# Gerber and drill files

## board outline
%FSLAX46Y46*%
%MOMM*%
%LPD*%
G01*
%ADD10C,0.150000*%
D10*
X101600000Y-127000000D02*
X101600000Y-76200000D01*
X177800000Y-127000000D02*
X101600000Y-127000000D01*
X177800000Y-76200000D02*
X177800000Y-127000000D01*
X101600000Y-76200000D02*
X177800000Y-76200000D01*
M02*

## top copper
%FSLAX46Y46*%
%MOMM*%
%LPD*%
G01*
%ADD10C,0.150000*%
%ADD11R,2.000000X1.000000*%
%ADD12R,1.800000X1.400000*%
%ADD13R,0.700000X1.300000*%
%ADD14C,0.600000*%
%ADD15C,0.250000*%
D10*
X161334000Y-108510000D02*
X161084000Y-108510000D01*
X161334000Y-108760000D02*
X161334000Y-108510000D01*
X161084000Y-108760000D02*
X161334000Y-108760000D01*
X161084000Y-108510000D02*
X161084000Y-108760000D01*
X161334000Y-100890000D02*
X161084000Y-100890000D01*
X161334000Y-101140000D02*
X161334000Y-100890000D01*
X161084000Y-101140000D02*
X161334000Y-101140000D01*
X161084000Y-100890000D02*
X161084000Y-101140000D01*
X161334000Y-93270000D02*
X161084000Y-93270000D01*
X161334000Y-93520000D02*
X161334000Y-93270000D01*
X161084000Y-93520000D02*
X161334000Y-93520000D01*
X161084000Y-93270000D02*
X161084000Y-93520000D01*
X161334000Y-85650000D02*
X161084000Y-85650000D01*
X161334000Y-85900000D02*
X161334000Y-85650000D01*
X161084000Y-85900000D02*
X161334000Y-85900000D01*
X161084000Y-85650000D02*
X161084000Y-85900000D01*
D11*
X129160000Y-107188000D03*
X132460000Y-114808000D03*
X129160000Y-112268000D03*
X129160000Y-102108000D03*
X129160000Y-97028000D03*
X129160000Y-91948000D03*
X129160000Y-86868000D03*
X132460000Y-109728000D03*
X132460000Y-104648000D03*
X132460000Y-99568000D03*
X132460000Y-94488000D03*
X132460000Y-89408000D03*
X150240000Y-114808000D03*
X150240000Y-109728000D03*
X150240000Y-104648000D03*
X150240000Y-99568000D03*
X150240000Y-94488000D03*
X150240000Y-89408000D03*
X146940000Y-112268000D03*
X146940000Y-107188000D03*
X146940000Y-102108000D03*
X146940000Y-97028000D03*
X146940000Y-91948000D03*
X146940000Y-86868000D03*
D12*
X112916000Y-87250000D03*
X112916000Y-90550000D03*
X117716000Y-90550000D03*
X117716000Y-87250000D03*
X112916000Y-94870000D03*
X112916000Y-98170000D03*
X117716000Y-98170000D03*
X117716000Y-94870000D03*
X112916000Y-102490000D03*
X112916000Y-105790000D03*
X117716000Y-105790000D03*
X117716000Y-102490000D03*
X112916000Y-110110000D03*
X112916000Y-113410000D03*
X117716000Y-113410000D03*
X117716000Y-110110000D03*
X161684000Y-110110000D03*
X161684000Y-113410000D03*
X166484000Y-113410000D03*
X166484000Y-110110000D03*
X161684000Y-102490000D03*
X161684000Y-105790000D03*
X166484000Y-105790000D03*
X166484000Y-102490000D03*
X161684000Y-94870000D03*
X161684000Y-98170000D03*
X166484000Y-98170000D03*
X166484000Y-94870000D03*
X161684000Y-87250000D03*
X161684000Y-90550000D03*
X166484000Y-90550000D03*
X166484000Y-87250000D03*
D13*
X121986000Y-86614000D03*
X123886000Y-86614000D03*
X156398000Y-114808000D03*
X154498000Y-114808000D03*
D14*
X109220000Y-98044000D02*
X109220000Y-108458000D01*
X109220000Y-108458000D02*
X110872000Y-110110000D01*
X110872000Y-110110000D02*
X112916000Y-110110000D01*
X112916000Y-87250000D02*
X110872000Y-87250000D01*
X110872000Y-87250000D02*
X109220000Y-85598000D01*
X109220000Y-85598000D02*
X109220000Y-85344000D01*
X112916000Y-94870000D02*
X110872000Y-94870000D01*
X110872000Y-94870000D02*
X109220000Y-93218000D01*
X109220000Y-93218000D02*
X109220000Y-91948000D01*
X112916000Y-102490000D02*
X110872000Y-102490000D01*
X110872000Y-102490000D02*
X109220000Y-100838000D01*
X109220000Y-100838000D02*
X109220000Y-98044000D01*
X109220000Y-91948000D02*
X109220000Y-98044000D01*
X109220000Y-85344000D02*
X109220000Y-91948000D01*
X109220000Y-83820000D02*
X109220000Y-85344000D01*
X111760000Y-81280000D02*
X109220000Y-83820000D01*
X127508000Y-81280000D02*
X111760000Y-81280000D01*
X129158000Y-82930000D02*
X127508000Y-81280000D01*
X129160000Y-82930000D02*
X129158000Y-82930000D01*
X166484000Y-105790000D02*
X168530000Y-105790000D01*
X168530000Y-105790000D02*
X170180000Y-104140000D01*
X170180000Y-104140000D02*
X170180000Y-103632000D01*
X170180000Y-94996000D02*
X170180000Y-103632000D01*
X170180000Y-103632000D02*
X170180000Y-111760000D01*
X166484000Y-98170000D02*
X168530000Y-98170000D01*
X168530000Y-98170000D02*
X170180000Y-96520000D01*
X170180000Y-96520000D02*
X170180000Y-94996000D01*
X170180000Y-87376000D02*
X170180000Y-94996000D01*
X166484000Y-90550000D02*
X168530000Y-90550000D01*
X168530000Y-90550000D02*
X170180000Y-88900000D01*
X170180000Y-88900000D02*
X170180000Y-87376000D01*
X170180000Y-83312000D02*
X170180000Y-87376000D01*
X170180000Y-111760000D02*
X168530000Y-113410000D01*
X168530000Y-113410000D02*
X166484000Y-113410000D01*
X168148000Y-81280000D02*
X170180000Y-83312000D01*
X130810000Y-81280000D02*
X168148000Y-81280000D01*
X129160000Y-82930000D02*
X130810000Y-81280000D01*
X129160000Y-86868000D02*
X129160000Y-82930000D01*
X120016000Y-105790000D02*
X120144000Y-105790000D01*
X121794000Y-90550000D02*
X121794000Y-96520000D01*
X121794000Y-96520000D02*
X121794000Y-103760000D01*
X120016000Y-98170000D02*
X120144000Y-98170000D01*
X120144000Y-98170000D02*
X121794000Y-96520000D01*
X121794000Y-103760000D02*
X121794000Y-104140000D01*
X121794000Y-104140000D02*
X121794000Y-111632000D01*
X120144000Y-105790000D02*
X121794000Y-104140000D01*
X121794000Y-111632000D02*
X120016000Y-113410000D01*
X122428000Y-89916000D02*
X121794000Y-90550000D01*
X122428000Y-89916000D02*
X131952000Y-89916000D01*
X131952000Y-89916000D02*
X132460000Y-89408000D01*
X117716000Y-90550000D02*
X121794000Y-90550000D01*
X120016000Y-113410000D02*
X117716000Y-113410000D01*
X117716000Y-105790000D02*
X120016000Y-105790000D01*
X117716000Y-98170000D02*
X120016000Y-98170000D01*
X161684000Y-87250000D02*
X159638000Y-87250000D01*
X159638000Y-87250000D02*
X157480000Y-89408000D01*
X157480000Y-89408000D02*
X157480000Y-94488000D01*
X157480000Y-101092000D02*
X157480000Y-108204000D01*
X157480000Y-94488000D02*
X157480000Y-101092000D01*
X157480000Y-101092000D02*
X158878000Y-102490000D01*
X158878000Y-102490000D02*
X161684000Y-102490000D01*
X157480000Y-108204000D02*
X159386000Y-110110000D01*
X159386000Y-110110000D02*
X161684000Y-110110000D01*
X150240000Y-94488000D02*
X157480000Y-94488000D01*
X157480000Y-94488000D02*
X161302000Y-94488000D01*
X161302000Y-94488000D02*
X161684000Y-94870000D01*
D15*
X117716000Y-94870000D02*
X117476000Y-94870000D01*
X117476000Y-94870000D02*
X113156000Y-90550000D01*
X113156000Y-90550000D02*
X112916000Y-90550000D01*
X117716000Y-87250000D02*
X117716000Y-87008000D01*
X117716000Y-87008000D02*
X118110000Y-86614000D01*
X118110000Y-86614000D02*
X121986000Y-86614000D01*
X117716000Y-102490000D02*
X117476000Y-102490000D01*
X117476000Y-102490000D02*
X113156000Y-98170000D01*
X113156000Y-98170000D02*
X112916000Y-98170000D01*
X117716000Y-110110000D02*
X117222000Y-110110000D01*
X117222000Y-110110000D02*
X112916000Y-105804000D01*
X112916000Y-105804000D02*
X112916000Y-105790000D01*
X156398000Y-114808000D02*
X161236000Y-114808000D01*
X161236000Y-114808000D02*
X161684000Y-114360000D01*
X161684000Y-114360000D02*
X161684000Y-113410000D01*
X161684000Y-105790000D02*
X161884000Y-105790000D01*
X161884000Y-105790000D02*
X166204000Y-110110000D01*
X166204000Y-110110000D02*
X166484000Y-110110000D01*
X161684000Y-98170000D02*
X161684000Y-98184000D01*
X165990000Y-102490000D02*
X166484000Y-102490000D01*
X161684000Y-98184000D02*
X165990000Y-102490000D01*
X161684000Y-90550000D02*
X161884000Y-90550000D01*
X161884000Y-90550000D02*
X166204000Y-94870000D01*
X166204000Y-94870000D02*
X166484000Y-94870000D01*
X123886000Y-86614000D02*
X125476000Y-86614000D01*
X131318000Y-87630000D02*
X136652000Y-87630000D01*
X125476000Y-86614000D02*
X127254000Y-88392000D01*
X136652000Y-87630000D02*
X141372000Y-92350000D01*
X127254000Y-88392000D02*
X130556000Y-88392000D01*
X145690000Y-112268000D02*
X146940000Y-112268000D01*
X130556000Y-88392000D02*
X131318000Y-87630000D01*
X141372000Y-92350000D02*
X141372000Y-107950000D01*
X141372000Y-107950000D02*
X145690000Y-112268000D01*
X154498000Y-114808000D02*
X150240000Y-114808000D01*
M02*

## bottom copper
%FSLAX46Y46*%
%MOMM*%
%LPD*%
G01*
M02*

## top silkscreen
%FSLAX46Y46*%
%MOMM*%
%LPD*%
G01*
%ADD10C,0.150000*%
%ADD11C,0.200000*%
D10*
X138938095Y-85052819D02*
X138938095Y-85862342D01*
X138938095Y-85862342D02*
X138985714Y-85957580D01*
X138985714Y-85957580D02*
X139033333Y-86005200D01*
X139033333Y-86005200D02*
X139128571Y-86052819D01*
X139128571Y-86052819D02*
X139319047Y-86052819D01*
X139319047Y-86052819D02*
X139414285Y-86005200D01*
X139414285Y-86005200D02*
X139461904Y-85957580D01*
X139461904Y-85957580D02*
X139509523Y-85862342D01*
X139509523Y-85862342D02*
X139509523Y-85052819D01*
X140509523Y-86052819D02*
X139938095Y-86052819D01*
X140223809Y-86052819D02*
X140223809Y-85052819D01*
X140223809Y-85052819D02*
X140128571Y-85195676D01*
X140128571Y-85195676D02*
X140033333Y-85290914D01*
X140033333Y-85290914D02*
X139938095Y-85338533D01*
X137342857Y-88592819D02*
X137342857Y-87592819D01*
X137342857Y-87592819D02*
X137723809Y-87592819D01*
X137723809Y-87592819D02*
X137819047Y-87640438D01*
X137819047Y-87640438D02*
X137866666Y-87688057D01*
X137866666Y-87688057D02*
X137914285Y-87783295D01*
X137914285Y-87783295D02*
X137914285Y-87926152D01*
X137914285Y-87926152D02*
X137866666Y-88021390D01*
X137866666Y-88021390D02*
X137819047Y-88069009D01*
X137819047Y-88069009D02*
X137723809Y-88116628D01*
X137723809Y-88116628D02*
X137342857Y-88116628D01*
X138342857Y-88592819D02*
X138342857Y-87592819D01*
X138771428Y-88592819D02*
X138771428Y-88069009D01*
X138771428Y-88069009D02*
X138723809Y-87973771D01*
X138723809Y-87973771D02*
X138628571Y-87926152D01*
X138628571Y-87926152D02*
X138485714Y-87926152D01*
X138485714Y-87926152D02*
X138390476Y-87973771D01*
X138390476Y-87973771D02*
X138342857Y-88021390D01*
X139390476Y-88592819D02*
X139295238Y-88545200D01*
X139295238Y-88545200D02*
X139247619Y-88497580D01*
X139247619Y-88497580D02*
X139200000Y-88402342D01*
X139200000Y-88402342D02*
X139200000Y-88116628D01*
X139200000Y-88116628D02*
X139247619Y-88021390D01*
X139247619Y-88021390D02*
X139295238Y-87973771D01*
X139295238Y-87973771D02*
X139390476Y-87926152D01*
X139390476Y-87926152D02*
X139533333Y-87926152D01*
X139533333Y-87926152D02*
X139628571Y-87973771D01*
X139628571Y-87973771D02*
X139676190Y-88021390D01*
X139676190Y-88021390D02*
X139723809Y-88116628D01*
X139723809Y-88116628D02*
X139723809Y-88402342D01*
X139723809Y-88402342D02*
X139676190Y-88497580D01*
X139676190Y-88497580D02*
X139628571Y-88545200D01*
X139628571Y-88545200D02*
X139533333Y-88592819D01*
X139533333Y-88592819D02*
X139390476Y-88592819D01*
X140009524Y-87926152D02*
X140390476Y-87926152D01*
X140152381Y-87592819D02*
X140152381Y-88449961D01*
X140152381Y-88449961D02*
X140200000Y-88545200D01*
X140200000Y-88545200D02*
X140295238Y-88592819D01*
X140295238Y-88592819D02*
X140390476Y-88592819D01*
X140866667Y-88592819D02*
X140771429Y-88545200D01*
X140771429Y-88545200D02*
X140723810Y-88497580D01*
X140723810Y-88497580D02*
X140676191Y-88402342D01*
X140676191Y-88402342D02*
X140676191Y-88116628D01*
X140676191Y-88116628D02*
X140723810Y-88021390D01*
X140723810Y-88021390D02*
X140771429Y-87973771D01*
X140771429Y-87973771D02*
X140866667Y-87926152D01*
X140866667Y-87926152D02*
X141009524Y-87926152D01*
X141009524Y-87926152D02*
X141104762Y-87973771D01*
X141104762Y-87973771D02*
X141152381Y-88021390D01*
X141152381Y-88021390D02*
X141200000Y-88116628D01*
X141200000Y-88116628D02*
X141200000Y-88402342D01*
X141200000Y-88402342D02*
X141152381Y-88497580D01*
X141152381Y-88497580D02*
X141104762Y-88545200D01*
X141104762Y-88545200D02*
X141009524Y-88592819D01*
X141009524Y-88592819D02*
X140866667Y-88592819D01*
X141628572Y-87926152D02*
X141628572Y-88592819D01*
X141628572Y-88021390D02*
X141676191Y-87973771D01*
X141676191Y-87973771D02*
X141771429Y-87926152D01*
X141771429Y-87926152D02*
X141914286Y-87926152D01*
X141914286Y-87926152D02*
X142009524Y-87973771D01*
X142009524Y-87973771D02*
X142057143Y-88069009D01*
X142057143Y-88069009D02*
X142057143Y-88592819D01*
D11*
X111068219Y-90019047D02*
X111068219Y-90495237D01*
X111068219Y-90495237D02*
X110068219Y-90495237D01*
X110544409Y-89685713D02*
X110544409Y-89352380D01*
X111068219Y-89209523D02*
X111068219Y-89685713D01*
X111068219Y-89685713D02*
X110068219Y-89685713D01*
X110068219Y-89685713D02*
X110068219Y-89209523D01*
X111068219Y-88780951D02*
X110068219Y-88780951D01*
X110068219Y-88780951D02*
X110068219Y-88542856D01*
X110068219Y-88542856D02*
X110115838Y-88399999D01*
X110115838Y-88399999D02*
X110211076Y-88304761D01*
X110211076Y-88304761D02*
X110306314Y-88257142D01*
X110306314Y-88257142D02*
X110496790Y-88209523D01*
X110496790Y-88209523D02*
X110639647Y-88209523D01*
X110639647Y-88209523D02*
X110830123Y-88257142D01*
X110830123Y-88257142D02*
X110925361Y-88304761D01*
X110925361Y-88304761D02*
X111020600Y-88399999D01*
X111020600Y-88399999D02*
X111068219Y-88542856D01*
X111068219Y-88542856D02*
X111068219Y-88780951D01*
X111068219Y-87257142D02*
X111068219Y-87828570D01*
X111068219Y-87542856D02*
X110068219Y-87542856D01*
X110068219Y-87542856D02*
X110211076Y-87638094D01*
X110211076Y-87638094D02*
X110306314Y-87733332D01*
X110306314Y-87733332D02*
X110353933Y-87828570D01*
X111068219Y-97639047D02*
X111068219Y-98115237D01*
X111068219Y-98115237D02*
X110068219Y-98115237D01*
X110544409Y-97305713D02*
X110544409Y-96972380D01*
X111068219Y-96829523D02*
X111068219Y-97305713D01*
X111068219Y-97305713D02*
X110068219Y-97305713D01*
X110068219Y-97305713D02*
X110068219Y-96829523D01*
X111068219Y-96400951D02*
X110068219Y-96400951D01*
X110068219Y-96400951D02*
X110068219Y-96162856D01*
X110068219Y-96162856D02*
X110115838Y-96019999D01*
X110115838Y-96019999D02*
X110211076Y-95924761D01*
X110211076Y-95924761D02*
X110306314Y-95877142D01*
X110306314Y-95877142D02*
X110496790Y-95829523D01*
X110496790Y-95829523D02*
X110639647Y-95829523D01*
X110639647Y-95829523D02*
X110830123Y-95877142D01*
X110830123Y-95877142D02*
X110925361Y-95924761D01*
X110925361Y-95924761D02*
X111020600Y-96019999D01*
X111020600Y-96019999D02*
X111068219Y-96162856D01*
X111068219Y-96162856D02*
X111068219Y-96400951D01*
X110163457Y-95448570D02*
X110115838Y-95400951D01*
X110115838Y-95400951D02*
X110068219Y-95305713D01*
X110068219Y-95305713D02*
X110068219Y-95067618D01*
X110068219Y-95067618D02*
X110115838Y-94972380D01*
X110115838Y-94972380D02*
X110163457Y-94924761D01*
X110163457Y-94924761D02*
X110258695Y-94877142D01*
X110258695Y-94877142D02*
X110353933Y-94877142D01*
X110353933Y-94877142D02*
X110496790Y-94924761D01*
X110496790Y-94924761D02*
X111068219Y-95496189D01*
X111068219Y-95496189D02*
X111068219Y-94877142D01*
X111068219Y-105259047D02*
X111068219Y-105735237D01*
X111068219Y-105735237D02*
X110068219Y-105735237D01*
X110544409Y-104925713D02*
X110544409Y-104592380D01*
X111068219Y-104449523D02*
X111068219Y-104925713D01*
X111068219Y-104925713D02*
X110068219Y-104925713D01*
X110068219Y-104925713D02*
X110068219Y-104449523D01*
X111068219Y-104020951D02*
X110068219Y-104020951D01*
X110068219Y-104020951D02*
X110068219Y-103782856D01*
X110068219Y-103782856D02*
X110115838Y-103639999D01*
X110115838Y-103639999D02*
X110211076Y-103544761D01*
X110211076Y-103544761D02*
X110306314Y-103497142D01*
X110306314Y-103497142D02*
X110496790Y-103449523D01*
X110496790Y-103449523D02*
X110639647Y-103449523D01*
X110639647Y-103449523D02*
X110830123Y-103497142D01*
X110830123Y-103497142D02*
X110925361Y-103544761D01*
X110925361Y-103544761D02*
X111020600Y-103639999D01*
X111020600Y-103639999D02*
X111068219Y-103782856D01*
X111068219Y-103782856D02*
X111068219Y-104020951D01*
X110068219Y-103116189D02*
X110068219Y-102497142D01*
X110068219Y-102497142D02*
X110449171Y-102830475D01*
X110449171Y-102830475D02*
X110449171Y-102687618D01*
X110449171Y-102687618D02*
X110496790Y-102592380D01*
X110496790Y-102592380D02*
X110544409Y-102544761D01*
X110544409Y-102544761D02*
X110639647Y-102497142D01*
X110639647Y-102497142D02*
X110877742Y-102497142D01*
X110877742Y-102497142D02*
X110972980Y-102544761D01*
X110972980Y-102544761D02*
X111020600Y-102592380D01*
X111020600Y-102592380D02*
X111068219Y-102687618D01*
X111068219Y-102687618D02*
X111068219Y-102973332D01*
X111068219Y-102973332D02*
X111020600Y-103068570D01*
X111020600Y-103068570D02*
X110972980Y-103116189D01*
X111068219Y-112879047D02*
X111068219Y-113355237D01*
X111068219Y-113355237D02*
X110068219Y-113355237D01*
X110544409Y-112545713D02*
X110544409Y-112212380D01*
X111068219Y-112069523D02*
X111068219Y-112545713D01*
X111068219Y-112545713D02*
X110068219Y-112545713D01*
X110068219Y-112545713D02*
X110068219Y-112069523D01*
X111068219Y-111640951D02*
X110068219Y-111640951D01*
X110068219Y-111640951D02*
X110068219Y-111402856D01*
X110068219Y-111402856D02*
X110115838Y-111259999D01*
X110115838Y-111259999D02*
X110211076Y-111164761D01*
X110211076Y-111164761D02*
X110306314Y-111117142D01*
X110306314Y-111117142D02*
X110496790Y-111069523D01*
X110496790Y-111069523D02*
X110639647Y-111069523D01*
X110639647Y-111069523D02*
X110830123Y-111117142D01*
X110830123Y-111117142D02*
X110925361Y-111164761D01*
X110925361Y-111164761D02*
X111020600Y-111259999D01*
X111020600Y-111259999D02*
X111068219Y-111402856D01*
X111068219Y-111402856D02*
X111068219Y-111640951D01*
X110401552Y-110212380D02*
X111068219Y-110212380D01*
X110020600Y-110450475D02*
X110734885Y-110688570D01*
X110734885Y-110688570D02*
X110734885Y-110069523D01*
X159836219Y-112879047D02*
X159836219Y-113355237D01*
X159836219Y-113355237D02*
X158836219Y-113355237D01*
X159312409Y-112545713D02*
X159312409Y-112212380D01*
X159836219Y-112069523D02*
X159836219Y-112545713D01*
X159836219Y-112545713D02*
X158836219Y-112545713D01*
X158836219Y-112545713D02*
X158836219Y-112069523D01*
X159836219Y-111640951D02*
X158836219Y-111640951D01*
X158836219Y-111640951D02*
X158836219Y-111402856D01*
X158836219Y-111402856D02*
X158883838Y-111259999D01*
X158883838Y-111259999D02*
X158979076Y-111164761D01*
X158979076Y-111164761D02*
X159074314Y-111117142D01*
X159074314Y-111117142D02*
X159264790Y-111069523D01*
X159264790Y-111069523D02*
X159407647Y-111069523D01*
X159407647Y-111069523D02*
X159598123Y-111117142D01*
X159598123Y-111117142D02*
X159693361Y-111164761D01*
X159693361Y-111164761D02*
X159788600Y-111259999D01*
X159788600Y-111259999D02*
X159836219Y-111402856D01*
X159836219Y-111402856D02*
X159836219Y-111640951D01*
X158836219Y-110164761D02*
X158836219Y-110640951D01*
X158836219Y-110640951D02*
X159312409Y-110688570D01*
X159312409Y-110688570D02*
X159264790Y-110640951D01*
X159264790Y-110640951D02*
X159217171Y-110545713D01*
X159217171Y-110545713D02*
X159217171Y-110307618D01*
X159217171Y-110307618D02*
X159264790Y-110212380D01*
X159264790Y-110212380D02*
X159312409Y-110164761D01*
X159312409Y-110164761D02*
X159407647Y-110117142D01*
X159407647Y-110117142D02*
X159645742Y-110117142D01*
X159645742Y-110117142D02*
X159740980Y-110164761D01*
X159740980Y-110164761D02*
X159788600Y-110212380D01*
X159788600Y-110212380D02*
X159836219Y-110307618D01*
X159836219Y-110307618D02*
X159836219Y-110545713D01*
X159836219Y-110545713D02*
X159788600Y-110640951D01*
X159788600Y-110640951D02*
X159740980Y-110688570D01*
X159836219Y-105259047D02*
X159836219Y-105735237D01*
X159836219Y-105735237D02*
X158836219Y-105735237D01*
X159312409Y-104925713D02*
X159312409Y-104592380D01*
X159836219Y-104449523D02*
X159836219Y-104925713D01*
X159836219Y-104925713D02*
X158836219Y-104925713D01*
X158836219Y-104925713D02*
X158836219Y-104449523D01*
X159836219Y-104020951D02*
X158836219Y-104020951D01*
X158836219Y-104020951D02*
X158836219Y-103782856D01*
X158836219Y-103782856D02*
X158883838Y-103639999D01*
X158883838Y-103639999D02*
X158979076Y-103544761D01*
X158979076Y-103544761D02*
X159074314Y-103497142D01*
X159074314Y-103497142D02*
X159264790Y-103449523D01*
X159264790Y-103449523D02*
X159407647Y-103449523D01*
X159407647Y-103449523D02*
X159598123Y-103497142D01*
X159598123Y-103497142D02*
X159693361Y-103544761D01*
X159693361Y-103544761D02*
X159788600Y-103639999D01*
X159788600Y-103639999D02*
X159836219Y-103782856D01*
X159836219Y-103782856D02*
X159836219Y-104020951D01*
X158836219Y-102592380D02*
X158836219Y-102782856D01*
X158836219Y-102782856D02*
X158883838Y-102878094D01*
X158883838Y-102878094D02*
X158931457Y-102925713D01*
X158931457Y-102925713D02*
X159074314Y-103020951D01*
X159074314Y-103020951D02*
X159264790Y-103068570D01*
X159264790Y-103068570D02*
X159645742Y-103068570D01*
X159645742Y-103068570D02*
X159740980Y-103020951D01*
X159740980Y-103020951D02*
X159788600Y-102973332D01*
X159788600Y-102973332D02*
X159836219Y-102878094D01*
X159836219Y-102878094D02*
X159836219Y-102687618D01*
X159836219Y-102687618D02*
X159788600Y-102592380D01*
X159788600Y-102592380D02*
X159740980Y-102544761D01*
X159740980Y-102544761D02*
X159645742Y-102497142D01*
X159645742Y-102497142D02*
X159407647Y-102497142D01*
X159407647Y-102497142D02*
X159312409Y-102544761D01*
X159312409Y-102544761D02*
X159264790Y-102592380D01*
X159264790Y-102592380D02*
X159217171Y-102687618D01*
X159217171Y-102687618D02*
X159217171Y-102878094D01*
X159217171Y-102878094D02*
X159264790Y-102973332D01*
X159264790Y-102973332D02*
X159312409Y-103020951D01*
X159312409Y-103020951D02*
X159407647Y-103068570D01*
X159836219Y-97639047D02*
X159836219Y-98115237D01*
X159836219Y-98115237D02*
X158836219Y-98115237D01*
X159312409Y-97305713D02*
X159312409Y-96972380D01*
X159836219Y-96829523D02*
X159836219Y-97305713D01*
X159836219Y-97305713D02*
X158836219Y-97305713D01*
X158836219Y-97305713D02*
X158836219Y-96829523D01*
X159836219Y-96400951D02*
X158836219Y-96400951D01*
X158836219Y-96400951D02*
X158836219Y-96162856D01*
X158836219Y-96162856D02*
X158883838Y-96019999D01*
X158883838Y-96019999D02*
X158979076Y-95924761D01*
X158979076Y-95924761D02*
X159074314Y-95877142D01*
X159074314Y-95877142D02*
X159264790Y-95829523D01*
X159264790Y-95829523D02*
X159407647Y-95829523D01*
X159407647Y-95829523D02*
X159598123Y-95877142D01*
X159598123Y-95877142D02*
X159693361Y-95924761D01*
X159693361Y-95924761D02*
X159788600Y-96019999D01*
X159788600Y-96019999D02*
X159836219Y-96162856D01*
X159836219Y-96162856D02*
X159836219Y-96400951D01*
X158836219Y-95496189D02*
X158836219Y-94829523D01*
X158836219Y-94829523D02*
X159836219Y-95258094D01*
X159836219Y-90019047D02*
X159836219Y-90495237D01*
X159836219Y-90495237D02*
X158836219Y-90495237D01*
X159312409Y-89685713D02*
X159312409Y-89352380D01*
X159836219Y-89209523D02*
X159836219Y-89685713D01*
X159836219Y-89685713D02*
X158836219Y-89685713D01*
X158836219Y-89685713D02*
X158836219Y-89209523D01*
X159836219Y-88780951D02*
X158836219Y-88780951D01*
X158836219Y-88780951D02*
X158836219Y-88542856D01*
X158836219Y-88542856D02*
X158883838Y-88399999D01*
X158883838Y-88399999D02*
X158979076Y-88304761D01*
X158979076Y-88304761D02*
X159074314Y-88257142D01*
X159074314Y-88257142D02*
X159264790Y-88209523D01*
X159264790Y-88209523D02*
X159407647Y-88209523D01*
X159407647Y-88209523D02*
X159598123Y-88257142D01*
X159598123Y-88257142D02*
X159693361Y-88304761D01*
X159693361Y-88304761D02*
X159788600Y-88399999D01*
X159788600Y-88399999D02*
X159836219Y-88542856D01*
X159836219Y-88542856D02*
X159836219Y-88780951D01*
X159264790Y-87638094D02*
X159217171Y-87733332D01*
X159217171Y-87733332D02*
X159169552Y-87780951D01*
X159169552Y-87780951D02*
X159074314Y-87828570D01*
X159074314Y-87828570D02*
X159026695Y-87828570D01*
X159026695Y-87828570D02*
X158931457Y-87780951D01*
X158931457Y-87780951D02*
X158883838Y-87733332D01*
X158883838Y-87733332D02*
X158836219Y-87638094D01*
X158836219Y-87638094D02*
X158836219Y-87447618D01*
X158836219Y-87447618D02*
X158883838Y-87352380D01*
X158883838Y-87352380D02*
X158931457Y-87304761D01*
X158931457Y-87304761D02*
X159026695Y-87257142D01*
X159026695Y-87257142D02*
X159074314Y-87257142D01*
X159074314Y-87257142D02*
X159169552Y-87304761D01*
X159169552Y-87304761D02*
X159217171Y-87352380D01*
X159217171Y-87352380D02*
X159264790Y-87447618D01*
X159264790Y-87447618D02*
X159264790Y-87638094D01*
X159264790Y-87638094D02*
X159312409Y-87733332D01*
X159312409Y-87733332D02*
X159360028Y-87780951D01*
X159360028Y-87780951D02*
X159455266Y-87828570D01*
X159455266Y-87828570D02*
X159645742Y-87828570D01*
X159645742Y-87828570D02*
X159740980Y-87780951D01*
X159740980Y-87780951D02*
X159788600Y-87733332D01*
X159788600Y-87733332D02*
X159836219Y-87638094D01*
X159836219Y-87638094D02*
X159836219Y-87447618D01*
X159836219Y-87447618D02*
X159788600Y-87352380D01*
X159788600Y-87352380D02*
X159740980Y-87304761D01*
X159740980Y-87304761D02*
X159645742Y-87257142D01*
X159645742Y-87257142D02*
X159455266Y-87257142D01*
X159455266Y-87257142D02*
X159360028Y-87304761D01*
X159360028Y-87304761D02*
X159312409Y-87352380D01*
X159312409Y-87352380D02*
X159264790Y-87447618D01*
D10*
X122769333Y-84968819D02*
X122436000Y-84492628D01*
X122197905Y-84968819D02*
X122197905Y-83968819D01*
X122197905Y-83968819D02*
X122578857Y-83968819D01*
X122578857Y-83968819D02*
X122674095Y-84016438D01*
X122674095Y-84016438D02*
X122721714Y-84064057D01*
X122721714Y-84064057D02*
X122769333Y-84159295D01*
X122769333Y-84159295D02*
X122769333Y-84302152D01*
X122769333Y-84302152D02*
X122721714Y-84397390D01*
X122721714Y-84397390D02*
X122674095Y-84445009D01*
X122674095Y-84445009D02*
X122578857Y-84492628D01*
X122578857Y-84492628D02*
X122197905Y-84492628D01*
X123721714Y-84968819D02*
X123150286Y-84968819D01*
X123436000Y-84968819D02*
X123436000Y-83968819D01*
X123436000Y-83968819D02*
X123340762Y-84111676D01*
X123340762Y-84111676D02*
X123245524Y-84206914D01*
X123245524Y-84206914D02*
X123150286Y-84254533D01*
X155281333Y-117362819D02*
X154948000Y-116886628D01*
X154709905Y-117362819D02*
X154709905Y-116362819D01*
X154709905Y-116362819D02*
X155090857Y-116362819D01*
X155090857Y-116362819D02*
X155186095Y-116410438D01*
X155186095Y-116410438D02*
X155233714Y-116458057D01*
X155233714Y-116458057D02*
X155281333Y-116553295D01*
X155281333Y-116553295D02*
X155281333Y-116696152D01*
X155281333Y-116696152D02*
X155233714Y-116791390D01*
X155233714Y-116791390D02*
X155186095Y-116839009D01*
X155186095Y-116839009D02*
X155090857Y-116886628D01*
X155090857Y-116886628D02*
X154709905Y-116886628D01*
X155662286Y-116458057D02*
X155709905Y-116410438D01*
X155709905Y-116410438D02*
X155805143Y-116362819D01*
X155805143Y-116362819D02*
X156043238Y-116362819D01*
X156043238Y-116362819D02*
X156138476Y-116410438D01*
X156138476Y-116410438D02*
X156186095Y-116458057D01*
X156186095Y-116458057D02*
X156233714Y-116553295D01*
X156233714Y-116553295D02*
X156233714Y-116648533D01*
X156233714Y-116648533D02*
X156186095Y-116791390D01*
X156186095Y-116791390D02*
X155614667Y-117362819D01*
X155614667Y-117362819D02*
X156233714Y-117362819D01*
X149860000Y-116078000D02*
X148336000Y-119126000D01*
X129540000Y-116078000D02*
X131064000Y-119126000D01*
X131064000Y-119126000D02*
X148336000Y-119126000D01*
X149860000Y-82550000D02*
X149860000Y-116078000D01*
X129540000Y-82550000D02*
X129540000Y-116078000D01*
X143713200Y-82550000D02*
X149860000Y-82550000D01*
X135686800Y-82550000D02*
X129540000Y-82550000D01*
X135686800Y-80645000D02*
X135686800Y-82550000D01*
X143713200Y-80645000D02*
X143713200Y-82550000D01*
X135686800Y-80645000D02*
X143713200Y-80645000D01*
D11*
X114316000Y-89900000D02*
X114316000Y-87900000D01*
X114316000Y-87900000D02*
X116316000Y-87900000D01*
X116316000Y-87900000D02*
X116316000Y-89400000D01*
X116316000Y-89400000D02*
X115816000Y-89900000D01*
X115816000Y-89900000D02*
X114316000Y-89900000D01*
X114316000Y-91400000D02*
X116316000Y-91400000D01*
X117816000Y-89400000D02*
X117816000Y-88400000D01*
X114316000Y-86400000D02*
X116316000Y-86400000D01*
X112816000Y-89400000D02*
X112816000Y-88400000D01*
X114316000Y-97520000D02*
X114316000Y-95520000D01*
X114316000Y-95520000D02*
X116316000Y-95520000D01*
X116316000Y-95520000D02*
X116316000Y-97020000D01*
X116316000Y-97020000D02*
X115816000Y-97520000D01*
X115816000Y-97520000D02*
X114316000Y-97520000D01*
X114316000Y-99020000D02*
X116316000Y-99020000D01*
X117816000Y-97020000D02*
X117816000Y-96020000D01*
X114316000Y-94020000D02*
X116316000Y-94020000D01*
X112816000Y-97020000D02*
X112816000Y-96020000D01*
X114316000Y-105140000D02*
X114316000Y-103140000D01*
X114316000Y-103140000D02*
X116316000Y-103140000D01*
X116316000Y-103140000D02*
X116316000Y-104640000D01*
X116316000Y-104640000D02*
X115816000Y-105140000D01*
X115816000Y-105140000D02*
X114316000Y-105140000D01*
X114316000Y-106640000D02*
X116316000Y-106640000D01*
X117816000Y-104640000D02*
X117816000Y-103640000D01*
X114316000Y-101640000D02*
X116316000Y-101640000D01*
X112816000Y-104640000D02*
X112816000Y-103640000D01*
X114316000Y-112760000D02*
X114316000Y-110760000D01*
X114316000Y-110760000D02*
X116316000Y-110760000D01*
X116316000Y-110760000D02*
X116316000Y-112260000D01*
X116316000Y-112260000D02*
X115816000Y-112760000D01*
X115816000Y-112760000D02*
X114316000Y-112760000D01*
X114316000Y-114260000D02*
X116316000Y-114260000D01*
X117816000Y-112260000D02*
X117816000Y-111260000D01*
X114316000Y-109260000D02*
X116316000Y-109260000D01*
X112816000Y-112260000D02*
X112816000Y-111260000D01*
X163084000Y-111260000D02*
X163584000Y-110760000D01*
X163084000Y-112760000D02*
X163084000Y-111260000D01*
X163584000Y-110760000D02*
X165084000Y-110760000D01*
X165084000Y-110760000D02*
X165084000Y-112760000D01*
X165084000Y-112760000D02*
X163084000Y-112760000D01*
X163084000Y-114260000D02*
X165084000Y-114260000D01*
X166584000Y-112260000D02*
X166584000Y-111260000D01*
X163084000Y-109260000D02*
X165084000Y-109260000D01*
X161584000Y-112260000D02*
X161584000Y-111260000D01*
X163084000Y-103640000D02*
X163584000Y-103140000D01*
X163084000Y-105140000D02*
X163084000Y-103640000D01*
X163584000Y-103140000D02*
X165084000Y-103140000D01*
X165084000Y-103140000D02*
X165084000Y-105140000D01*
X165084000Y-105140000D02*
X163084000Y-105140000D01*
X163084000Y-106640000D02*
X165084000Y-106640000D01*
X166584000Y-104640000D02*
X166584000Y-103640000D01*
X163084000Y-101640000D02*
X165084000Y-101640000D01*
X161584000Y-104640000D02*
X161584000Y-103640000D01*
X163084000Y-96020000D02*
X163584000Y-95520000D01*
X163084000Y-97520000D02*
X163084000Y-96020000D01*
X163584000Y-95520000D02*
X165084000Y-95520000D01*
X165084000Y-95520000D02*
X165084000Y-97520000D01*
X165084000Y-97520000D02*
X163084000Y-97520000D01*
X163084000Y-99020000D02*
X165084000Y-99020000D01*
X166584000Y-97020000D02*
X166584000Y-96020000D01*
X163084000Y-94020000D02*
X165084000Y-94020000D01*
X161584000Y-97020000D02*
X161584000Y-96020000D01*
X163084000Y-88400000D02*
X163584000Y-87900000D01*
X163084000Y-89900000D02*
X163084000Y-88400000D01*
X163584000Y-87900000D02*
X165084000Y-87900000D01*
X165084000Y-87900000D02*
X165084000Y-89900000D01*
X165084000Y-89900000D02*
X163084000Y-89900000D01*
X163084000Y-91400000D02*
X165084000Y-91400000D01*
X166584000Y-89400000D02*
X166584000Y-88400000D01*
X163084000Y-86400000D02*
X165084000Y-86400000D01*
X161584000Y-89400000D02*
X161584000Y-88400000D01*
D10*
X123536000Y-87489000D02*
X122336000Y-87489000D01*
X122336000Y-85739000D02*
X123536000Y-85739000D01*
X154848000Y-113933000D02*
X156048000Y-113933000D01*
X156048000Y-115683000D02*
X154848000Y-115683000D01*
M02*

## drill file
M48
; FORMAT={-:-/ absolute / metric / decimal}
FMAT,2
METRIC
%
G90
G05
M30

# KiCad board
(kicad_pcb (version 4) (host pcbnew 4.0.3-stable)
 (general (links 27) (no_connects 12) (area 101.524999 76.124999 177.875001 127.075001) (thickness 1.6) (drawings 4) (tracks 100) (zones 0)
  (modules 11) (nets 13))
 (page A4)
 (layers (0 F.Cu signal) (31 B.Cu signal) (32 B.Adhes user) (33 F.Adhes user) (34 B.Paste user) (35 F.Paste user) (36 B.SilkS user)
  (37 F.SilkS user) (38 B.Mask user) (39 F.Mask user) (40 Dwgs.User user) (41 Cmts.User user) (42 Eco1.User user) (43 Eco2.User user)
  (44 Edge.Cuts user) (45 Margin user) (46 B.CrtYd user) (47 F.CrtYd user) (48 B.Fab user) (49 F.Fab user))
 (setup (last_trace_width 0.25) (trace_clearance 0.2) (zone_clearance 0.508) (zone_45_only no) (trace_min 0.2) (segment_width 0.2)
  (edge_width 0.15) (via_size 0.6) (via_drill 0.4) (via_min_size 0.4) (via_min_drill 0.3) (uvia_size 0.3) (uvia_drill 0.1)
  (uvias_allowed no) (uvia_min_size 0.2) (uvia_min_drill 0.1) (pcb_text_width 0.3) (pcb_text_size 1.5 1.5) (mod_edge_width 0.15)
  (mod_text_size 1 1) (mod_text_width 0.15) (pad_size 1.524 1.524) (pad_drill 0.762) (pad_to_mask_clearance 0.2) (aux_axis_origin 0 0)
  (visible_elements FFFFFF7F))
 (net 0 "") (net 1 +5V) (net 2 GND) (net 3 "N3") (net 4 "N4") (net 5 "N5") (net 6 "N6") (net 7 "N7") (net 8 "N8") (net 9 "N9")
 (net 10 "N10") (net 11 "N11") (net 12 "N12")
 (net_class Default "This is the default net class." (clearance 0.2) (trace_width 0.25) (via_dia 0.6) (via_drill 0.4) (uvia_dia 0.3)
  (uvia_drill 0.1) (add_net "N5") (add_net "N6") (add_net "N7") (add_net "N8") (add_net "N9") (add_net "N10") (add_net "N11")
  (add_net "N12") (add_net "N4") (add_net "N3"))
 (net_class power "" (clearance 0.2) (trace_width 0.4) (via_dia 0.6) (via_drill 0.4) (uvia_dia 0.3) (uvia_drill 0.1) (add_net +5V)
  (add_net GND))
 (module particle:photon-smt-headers (layer F.Cu) (at 139.7 102.108)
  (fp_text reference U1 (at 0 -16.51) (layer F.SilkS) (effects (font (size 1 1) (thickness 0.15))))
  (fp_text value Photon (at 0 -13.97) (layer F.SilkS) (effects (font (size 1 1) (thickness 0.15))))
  (fp_line (start 10.16 13.97) (end 8.636 17.018) (layer F.SilkS) (width 0.15))
  (fp_line (start -10.16 13.97) (end -8.636 17.018) (layer F.SilkS) (width 0.15))
  (fp_line (start -8.636 17.018) (end 8.636 17.018) (layer F.SilkS) (width 0.15))
  (fp_line (start 10.16 -19.558) (end 10.16 13.97) (layer F.SilkS) (width 0.15))
  (fp_line (start -10.16 -19.558) (end -10.16 13.97) (layer F.SilkS) (width 0.15))
  (fp_line (start 4.0132 -19.558) (end 10.16 -19.558) (layer F.SilkS) (width 0.15))
  (fp_line (start -4.0132 -19.558) (end -10.16 -19.558) (layer F.SilkS) (width 0.15))
  (fp_line (start -4.0132 -21.463) (end -4.0132 -19.558) (layer F.SilkS) (width 0.15))
  (fp_line (start 4.0132 -21.463) (end 4.0132 -19.558) (layer F.SilkS) (width 0.15))
  (fp_line (start -4.0132 -21.463) (end 4.0132 -21.463) (layer F.SilkS) (width 0.15))
  (pad 9 smd rect (at -10.54 5.08) (size 2 1) (layers F.Cu F.Paste F.Mask))
  (pad 12 smd rect (at -7.24 12.7) (size 2 1) (layers F.Cu F.Paste F.Mask))
  (pad 11 smd rect (at -10.54 10.16) (size 2 1) (layers F.Cu F.Paste F.Mask))
  (pad 7 smd rect (at -10.54 0) (size 2 1) (layers F.Cu F.Paste F.Mask))
  (pad 5 smd rect (at -10.54 -5.08) (size 2 1) (layers F.Cu F.Paste F.Mask))
  (pad 3 smd rect (at -10.54 -10.16) (size 2 1) (layers F.Cu F.Paste F.Mask))
  (pad 1 smd rect (at -10.54 -15.24) (size 2 1) (layers F.Cu F.Paste F.Mask) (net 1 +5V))
  (pad 10 smd rect (at -7.24 7.62) (size 2 1) (layers F.Cu F.Paste F.Mask))
  (pad 8 smd rect (at -7.24 2.54) (size 2 1) (layers F.Cu F.Paste F.Mask))
  (pad 6 smd rect (at -7.24 -2.54) (size 2 1) (layers F.Cu F.Paste F.Mask))
  (pad 4 smd rect (at -7.24 -7.62) (size 2 1) (layers F.Cu F.Paste F.Mask))
  (pad 2 smd rect (at -7.24 -12.7) (size 2 1) (layers F.Cu F.Paste F.Mask) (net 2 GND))
  (pad 13 smd rect (at 10.54 12.7) (size 2 1) (layers F.Cu F.Paste F.Mask) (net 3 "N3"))
  (pad 15 smd rect (at 10.54 7.62) (size 2 1) (layers F.Cu F.Paste F.Mask))
  (pad 17 smd rect (at 10.54 2.54) (size 2 1) (layers F.Cu F.Paste F.Mask))
  (pad 19 smd rect (at 10.54 -2.54) (size 2 1) (layers F.Cu F.Paste F.Mask))
  (pad 21 smd rect (at 10.54 -7.62) (size 2 1) (layers F.Cu F.Paste F.Mask) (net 2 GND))
  (pad 23 smd rect (at 10.54 -12.7) (size 2 1) (layers F.Cu F.Paste F.Mask))
  (pad 14 smd rect (at 7.24 10.16) (size 2 1) (layers F.Cu F.Paste F.Mask) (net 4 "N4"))
  (pad 16 smd rect (at 7.24 5.08) (size 2 1) (layers F.Cu F.Paste F.Mask))
  (pad 18 smd rect (at 7.24 0) (size 2 1) (layers F.Cu F.Paste F.Mask))
  (pad 20 smd rect (at 7.24 -5.08) (size 2 1) (layers F.Cu F.Paste F.Mask))
  (pad 22 smd rect (at 7.24 -10.16) (size 2 1) (layers F.Cu F.Paste F.Mask))
  (pad 24 smd rect (at 7.24 -15.24) (size 2 1) (layers F.Cu F.Paste F.Mask)))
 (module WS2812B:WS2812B (layer F.Cu) (at 115.316 88.9 90)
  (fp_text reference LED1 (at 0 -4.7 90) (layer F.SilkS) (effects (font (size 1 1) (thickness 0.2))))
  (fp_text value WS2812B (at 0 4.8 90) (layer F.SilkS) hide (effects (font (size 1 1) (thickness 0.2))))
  (fp_line (start -1 -1) (end 1 -1) (layer F.SilkS) (width 0.2)) (fp_line (start 1 -1) (end 1 1) (layer F.SilkS) (width 0.2))
  (fp_line (start 1 1) (end -0.5 1) (layer F.SilkS) (width 0.2))
  (fp_line (start -0.5 1) (end -1 0.5) (layer F.SilkS) (width 0.2))
  (fp_line (start -1 0.5) (end -1 -1) (layer F.SilkS) (width 0.2))
  (fp_line (start -2.5 -1) (end -2.5 1) (layer F.SilkS) (width 0.2))
  (fp_line (start -0.5 2.5) (end 0.5 2.5) (layer F.SilkS) (width 0.2))
  (fp_line (start 2.5 -1) (end 2.5 1) (layer F.SilkS) (width 0.2))
  (fp_line (start -0.5 -2.5) (end 0.5 -2.5) (layer F.SilkS) (width 0.2))
  (pad 1 smd rect (at 1.65 -2.4 90) (size 1.4 1.8) (layers F.Cu F.Paste F.Mask) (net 1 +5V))
  (pad 2 smd rect (at -1.65 -2.4 90) (size 1.4 1.8) (layers F.Cu F.Paste F.Mask) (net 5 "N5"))
  (pad 3 smd rect (at -1.65 2.4 90) (size 1.4 1.8) (layers F.Cu F.Paste F.Mask) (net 2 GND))
  (pad 4 smd rect (at 1.65 2.4 90) (size 1.4 1.8) (layers F.Cu F.Paste F.Mask) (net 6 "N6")))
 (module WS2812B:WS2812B (layer F.Cu) (at 115.316 96.52 90)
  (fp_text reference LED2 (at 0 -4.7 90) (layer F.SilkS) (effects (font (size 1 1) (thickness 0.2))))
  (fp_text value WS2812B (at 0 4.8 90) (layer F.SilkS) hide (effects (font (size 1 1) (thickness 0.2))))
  (fp_line (start -1 -1) (end 1 -1) (layer F.SilkS) (width 0.2)) (fp_line (start 1 -1) (end 1 1) (layer F.SilkS) (width 0.2))
  (fp_line (start 1 1) (end -0.5 1) (layer F.SilkS) (width 0.2))
  (fp_line (start -0.5 1) (end -1 0.5) (layer F.SilkS) (width 0.2))
  (fp_line (start -1 0.5) (end -1 -1) (layer F.SilkS) (width 0.2))
  (fp_line (start -2.5 -1) (end -2.5 1) (layer F.SilkS) (width 0.2))
  (fp_line (start -0.5 2.5) (end 0.5 2.5) (layer F.SilkS) (width 0.2))
  (fp_line (start 2.5 -1) (end 2.5 1) (layer F.SilkS) (width 0.2))
  (fp_line (start -0.5 -2.5) (end 0.5 -2.5) (layer F.SilkS) (width 0.2))
  (pad 1 smd rect (at 1.65 -2.4 90) (size 1.4 1.8) (layers F.Cu F.Paste F.Mask) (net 1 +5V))
  (pad 2 smd rect (at -1.65 -2.4 90) (size 1.4 1.8) (layers F.Cu F.Paste F.Mask) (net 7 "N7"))
  (pad 3 smd rect (at -1.65 2.4 90) (size 1.4 1.8) (layers F.Cu F.Paste F.Mask) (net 2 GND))
  (pad 4 smd rect (at 1.65 2.4 90) (size 1.4 1.8) (layers F.Cu F.Paste F.Mask) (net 5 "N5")))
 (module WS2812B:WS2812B (layer F.Cu) (at 115.316 104.14 90)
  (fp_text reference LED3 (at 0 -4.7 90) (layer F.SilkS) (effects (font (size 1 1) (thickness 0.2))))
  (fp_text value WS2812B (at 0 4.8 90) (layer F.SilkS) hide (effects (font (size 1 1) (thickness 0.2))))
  (fp_line (start -1 -1) (end 1 -1) (layer F.SilkS) (width 0.2)) (fp_line (start 1 -1) (end 1 1) (layer F.SilkS) (width 0.2))
  (fp_line (start 1 1) (end -0.5 1) (layer F.SilkS) (width 0.2))
  (fp_line (start -0.5 1) (end -1 0.5) (layer F.SilkS) (width 0.2))
  (fp_line (start -1 0.5) (end -1 -1) (layer F.SilkS) (width 0.2))
  (fp_line (start -2.5 -1) (end -2.5 1) (layer F.SilkS) (width 0.2))
  (fp_line (start -0.5 2.5) (end 0.5 2.5) (layer F.SilkS) (width 0.2))
  (fp_line (start 2.5 -1) (end 2.5 1) (layer F.SilkS) (width 0.2))
  (fp_line (start -0.5 -2.5) (end 0.5 -2.5) (layer F.SilkS) (width 0.2))
  (pad 1 smd rect (at 1.65 -2.4 90) (size 1.4 1.8) (layers F.Cu F.Paste F.Mask) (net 1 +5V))
  (pad 2 smd rect (at -1.65 -2.4 90) (size 1.4 1.8) (layers F.Cu F.Paste F.Mask) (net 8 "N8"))
  (pad 3 smd rect (at -1.65 2.4 90) (size 1.4 1.8) (layers F.Cu F.Paste F.Mask) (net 2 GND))
  (pad 4 smd rect (at 1.65 2.4 90) (size 1.4 1.8) (layers F.Cu F.Paste F.Mask) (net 7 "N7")))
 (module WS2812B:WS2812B (layer F.Cu) (at 115.316 111.76 90)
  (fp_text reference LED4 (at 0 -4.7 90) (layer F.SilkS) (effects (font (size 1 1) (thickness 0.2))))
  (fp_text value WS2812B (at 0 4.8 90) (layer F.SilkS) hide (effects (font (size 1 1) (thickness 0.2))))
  (fp_line (start -1 -1) (end 1 -1) (layer F.SilkS) (width 0.2)) (fp_line (start 1 -1) (end 1 1) (layer F.SilkS) (width 0.2))
  (fp_line (start 1 1) (end -0.5 1) (layer F.SilkS) (width 0.2))
  (fp_line (start -0.5 1) (end -1 0.5) (layer F.SilkS) (width 0.2))
  (fp_line (start -1 0.5) (end -1 -1) (layer F.SilkS) (width 0.2))
  (fp_line (start -2.5 -1) (end -2.5 1) (layer F.SilkS) (width 0.2))
  (fp_line (start -0.5 2.5) (end 0.5 2.5) (layer F.SilkS) (width 0.2))
  (fp_line (start 2.5 -1) (end 2.5 1) (layer F.SilkS) (width 0.2))
  (fp_line (start -0.5 -2.5) (end 0.5 -2.5) (layer F.SilkS) (width 0.2))
  (pad 1 smd rect (at 1.65 -2.4 90) (size 1.4 1.8) (layers F.Cu F.Paste F.Mask) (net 1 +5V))
  (pad 2 smd rect (at -1.65 -2.4 90) (size 1.4 1.8) (layers F.Cu F.Paste F.Mask))
  (pad 3 smd rect (at -1.65 2.4 90) (size 1.4 1.8) (layers F.Cu F.Paste F.Mask) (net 2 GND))
  (pad 4 smd rect (at 1.65 2.4 90) (size 1.4 1.8) (layers F.Cu F.Paste F.Mask) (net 8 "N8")))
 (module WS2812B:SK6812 (layer F.Cu) (at 164.084 111.76 90)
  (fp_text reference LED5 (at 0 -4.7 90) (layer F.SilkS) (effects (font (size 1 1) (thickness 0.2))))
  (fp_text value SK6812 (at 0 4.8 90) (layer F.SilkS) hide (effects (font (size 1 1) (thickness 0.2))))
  (fp_line (start 3.25 -2.75) (end 3.25 -3) (layer F.Cu) (width 0.15))
  (fp_line (start 3 -2.75) (end 3.25 -2.75) (layer F.Cu) (width 0.15))
  (fp_line (start 3 -3) (end 3 -2.75) (layer F.Cu) (width 0.15))
  (fp_line (start 3.25 -3) (end 3 -3) (layer F.Cu) (width 0.15))
  (fp_line (start 0.5 -1) (end 1 -0.5) (layer F.SilkS) (width 0.2))
  (fp_line (start -1 -1) (end 0.5 -1) (layer F.SilkS) (width 0.2))
  (fp_line (start 1 -0.5) (end 1 1) (layer F.SilkS) (width 0.2)) (fp_line (start 1 1) (end -1 1) (layer F.SilkS) (width 0.2))
  (fp_line (start -1 1) (end -1 -1) (layer F.SilkS) (width 0.2))
  (fp_line (start -2.5 -1) (end -2.5 1) (layer F.SilkS) (width 0.2))
  (fp_line (start -0.5 2.5) (end 0.5 2.5) (layer F.SilkS) (width 0.2))
  (fp_line (start 2.5 -1) (end 2.5 1) (layer F.SilkS) (width 0.2))
  (fp_line (start -0.5 -2.5) (end 0.5 -2.5) (layer F.SilkS) (width 0.2))
  (pad 1 smd rect (at 1.65 -2.4 90) (size 1.4 1.8) (layers F.Cu F.Paste F.Mask) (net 2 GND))
  (pad 2 smd rect (at -1.65 -2.4 90) (size 1.4 1.8) (layers F.Cu F.Paste F.Mask) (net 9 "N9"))
  (pad 3 smd rect (at -1.65 2.4 90) (size 1.4 1.8) (layers F.Cu F.Paste F.Mask) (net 1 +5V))
  (pad 4 smd rect (at 1.65 2.4 90) (size 1.4 1.8) (layers F.Cu F.Paste F.Mask) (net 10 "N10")))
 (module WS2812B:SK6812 (layer F.Cu) (at 164.084 104.14 90)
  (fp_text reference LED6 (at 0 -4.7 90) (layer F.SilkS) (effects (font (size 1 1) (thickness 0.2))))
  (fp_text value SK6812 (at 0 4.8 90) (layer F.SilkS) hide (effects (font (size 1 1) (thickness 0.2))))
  (fp_line (start 3.25 -2.75) (end 3.25 -3) (layer F.Cu) (width 0.15))
  (fp_line (start 3 -2.75) (end 3.25 -2.75) (layer F.Cu) (width 0.15))
  (fp_line (start 3 -3) (end 3 -2.75) (layer F.Cu) (width 0.15))
  (fp_line (start 3.25 -3) (end 3 -3) (layer F.Cu) (width 0.15))
  (fp_line (start 0.5 -1) (end 1 -0.5) (layer F.SilkS) (width 0.2))
  (fp_line (start -1 -1) (end 0.5 -1) (layer F.SilkS) (width 0.2))
  (fp_line (start 1 -0.5) (end 1 1) (layer F.SilkS) (width 0.2)) (fp_line (start 1 1) (end -1 1) (layer F.SilkS) (width 0.2))
  (fp_line (start -1 1) (end -1 -1) (layer F.SilkS) (width 0.2))
  (fp_line (start -2.5 -1) (end -2.5 1) (layer F.SilkS) (width 0.2))
  (fp_line (start -0.5 2.5) (end 0.5 2.5) (layer F.SilkS) (width 0.2))
  (fp_line (start 2.5 -1) (end 2.5 1) (layer F.SilkS) (width 0.2))
  (fp_line (start -0.5 -2.5) (end 0.5 -2.5) (layer F.SilkS) (width 0.2))
  (pad 1 smd rect (at 1.65 -2.4 90) (size 1.4 1.8) (layers F.Cu F.Paste F.Mask) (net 2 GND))
  (pad 2 smd rect (at -1.65 -2.4 90) (size 1.4 1.8) (layers F.Cu F.Paste F.Mask) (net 10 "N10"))
  (pad 3 smd rect (at -1.65 2.4 90) (size 1.4 1.8) (layers F.Cu F.Paste F.Mask) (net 1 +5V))
  (pad 4 smd rect (at 1.65 2.4 90) (size 1.4 1.8) (layers F.Cu F.Paste F.Mask) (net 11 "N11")))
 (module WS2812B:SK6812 (layer F.Cu) (at 164.084 96.52 90)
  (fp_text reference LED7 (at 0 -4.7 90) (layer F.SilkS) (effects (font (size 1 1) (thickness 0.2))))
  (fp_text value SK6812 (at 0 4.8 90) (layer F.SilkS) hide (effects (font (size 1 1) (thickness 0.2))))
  (fp_line (start 3.25 -2.75) (end 3.25 -3) (layer F.Cu) (width 0.15))
  (fp_line (start 3 -2.75) (end 3.25 -2.75) (layer F.Cu) (width 0.15))
  (fp_line (start 3 -3) (end 3 -2.75) (layer F.Cu) (width 0.15))
  (fp_line (start 3.25 -3) (end 3 -3) (layer F.Cu) (width 0.15))
  (fp_line (start 0.5 -1) (end 1 -0.5) (layer F.SilkS) (width 0.2))
  (fp_line (start -1 -1) (end 0.5 -1) (layer F.SilkS) (width 0.2))
  (fp_line (start 1 -0.5) (end 1 1) (layer F.SilkS) (width 0.2)) (fp_line (start 1 1) (end -1 1) (layer F.SilkS) (width 0.2))
  (fp_line (start -1 1) (end -1 -1) (layer F.SilkS) (width 0.2))
  (fp_line (start -2.5 -1) (end -2.5 1) (layer F.SilkS) (width 0.2))
  (fp_line (start -0.5 2.5) (end 0.5 2.5) (layer F.SilkS) (width 0.2))
  (fp_line (start 2.5 -1) (end 2.5 1) (layer F.SilkS) (width 0.2))
  (fp_line (start -0.5 -2.5) (end 0.5 -2.5) (layer F.SilkS) (width 0.2))
  (pad 1 smd rect (at 1.65 -2.4 90) (size 1.4 1.8) (layers F.Cu F.Paste F.Mask) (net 2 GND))
  (pad 2 smd rect (at -1.65 -2.4 90) (size 1.4 1.8) (layers F.Cu F.Paste F.Mask) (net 11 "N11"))
  (pad 3 smd rect (at -1.65 2.4 90) (size 1.4 1.8) (layers F.Cu F.Paste F.Mask) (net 1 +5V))
  (pad 4 smd rect (at 1.65 2.4 90) (size 1.4 1.8) (layers F.Cu F.Paste F.Mask) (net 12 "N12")))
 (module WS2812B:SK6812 (layer F.Cu) (at 164.084 88.9 90)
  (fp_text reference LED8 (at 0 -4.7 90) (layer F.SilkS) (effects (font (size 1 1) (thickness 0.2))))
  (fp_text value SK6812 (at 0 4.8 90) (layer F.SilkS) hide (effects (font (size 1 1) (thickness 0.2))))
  (fp_line (start 3.25 -2.75) (end 3.25 -3) (layer F.Cu) (width 0.15))
  (fp_line (start 3 -2.75) (end 3.25 -2.75) (layer F.Cu) (width 0.15))
  (fp_line (start 3 -3) (end 3 -2.75) (layer F.Cu) (width 0.15))
  (fp_line (start 3.25 -3) (end 3 -3) (layer F.Cu) (width 0.15))
  (fp_line (start 0.5 -1) (end 1 -0.5) (layer F.SilkS) (width 0.2))
  (fp_line (start -1 -1) (end 0.5 -1) (layer F.SilkS) (width 0.2))
  (fp_line (start 1 -0.5) (end 1 1) (layer F.SilkS) (width 0.2)) (fp_line (start 1 1) (end -1 1) (layer F.SilkS) (width 0.2))
  (fp_line (start -1 1) (end -1 -1) (layer F.SilkS) (width 0.2))
  (fp_line (start -2.5 -1) (end -2.5 1) (layer F.SilkS) (width 0.2))
  (fp_line (start -0.5 2.5) (end 0.5 2.5) (layer F.SilkS) (width 0.2))
  (fp_line (start 2.5 -1) (end 2.5 1) (layer F.SilkS) (width 0.2))
  (fp_line (start -0.5 -2.5) (end 0.5 -2.5) (layer F.SilkS) (width 0.2))
  (pad 1 smd rect (at 1.65 -2.4 90) (size 1.4 1.8) (layers F.Cu F.Paste F.Mask) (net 2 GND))
  (pad 2 smd rect (at -1.65 -2.4 90) (size 1.4 1.8) (layers F.Cu F.Paste F.Mask) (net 12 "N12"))
  (pad 3 smd rect (at -1.65 2.4 90) (size 1.4 1.8) (layers F.Cu F.Paste F.Mask) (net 1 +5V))
  (pad 4 smd rect (at 1.65 2.4 90) (size 1.4 1.8) (layers F.Cu F.Paste F.Mask)))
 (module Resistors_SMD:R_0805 (layer F.Cu) (at 122.936 86.614)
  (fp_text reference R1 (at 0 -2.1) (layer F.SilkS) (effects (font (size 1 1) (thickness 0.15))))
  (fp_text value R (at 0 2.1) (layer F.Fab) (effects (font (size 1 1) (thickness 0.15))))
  (fp_line (start 0.6 0.875) (end -0.6 0.875) (layer F.SilkS) (width 0.15))
  (fp_line (start -0.6 -0.875) (end 0.6 -0.875) (layer F.SilkS) (width 0.15))
  (pad 1 smd rect (at -0.95 0) (size 0.7 1.3) (layers F.Cu F.Paste F.Mask) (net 6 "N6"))
  (pad 2 smd rect (at 0.95 0) (size 0.7 1.3) (layers F.Cu F.Paste F.Mask) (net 4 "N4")))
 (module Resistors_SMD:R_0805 (layer F.Cu) (at 155.448 114.808 180)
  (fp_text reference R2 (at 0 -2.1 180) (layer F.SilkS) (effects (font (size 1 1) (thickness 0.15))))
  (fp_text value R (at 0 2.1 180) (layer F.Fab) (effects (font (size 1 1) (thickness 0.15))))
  (fp_line (start 0.6 0.875) (end -0.6 0.875) (layer F.SilkS) (width 0.15))
  (fp_line (start -0.6 -0.875) (end 0.6 -0.875) (layer F.SilkS) (width 0.15))
  (pad 1 smd rect (at -0.95 0 180) (size 0.7 1.3) (layers F.Cu F.Paste F.Mask) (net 9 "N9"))
  (pad 2 smd rect (at 0.95 0 180) (size 0.7 1.3) (layers F.Cu F.Paste F.Mask) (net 3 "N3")))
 (gr_line (start 101.6 127) (end 101.6 76.2) (layer Edge.Cuts) (width 0.15))
 (gr_line (start 177.8 127) (end 101.6 127) (layer Edge.Cuts) (width 0.15))
 (gr_line (start 177.8 76.2) (end 177.8 127) (layer Edge.Cuts) (width 0.15))
 (gr_line (start 101.6 76.2) (end 177.8 76.2) (layer Edge.Cuts) (width 0.15))
 (segment (start 109.22 98.044) (end 109.22 108.458) (width 0.6) (layer F.Cu) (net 1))
 (segment (start 109.22 108.458) (end 110.872 110.11) (width 0.6) (layer F.Cu) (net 1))
 (segment (start 110.872 110.11) (end 112.916 110.11) (width 0.6) (layer F.Cu) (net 1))
 (segment (start 112.916 87.25) (end 110.872 87.25) (width 0.6) (layer F.Cu) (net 1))
 (segment (start 110.872 87.25) (end 109.22 85.598) (width 0.6) (layer F.Cu) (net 1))
 (segment (start 109.22 85.598) (end 109.22 85.344) (width 0.6) (layer F.Cu) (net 1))
 (segment (start 112.916 94.87) (end 110.872 94.87) (width 0.6) (layer F.Cu) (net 1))
 (segment (start 110.872 94.87) (end 109.22 93.218) (width 0.6) (layer F.Cu) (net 1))
 (segment (start 109.22 93.218) (end 109.22 91.948) (width 0.6) (layer F.Cu) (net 1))
 (segment (start 112.916 102.49) (end 110.872 102.49) (width 0.6) (layer F.Cu) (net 1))
 (segment (start 110.872 102.49) (end 109.22 100.838) (width 0.6) (layer F.Cu) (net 1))
 (segment (start 109.22 100.838) (end 109.22 98.044) (width 0.6) (layer F.Cu) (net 1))
 (segment (start 109.22 91.948) (end 109.22 98.044) (width 0.6) (layer F.Cu) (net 1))
 (segment (start 109.22 85.344) (end 109.22 91.948) (width 0.6) (layer F.Cu) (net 1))
 (segment (start 109.22 83.82) (end 109.22 85.344) (width 0.6) (layer F.Cu) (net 1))
 (segment (start 111.76 81.28) (end 109.22 83.82) (width 0.6) (layer F.Cu) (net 1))
 (segment (start 127.508 81.28) (end 111.76 81.28) (width 0.6) (layer F.Cu) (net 1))
 (segment (start 129.158 82.93) (end 127.508 81.28) (width 0.6) (layer F.Cu) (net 1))
 (segment (start 129.16 82.93) (end 129.158 82.93) (width 0.6) (layer F.Cu) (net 1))
 (segment (start 166.484 105.79) (end 168.53 105.79) (width 0.6) (layer F.Cu) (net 1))
 (segment (start 168.53 105.79) (end 170.18 104.14) (width 0.6) (layer F.Cu) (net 1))
 (segment (start 170.18 104.14) (end 170.18 103.632) (width 0.6) (layer F.Cu) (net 1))
 (segment (start 170.18 94.996) (end 170.18 103.632) (width 0.6) (layer F.Cu) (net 1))
 (segment (start 170.18 103.632) (end 170.18 111.76) (width 0.6) (layer F.Cu) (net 1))
 (segment (start 166.484 98.17) (end 168.53 98.17) (width 0.6) (layer F.Cu) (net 1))
 (segment (start 168.53 98.17) (end 170.18 96.52) (width 0.6) (layer F.Cu) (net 1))
 (segment (start 170.18 96.52) (end 170.18 94.996) (width 0.6) (layer F.Cu) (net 1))
 (segment (start 170.18 87.376) (end 170.18 94.996) (width 0.6) (layer F.Cu) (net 1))
 (segment (start 166.484 90.55) (end 168.53 90.55) (width 0.6) (layer F.Cu) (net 1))
 (segment (start 168.53 90.55) (end 170.18 88.9) (width 0.6) (layer F.Cu) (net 1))
 (segment (start 170.18 88.9) (end 170.18 87.376) (width 0.6) (layer F.Cu) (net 1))
 (segment (start 170.18 83.312) (end 170.18 87.376) (width 0.6) (layer F.Cu) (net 1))
 (segment (start 170.18 111.76) (end 168.53 113.41) (width 0.6) (layer F.Cu) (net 1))
 (segment (start 168.53 113.41) (end 166.484 113.41) (width 0.6) (layer F.Cu) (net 1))
 (segment (start 168.148 81.28) (end 170.18 83.312) (width 0.6) (layer F.Cu) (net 1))
 (segment (start 130.81 81.28) (end 168.148 81.28) (width 0.6) (layer F.Cu) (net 1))
 (segment (start 129.16 82.93) (end 130.81 81.28) (width 0.6) (layer F.Cu) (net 1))
 (segment (start 129.16 86.868) (end 129.16 82.93) (width 0.6) (layer F.Cu) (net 1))
 (segment (start 120.016 105.79) (end 120.144 105.79) (width 0.6) (layer F.Cu) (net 2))
 (segment (start 121.794 90.55) (end 121.794 96.52) (width 0.6) (layer F.Cu) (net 2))
 (segment (start 121.794 96.52) (end 121.794 103.76) (width 0.6) (layer F.Cu) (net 2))
 (segment (start 120.016 98.17) (end 120.144 98.17) (width 0.6) (layer F.Cu) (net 2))
 (segment (start 120.144 98.17) (end 121.794 96.52) (width 0.6) (layer F.Cu) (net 2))
 (segment (start 121.794 103.76) (end 121.794 104.14) (width 0.6) (layer F.Cu) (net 2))
 (segment (start 121.794 104.14) (end 121.794 111.632) (width 0.6) (layer F.Cu) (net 2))
 (segment (start 120.144 105.79) (end 121.794 104.14) (width 0.6) (layer F.Cu) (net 2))
 (segment (start 121.794 111.632) (end 120.016 113.41) (width 0.6) (layer F.Cu) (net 2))
 (segment (start 122.428 89.916) (end 121.794 90.55) (width 0.6) (layer F.Cu) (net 2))
 (segment (start 122.428 89.916) (end 131.952 89.916) (width 0.6) (layer F.Cu) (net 2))
 (segment (start 131.952 89.916) (end 132.46 89.408) (width 0.6) (layer F.Cu) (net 2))
 (segment (start 117.716 90.55) (end 121.794 90.55) (width 0.6) (layer F.Cu) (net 2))
 (segment (start 120.016 113.41) (end 117.716 113.41) (width 0.6) (layer F.Cu) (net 2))
 (segment (start 117.716 105.79) (end 120.016 105.79) (width 0.6) (layer F.Cu) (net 2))
 (segment (start 117.716 98.17) (end 120.016 98.17) (width 0.6) (layer F.Cu) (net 2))
 (segment (start 161.684 87.25) (end 159.638 87.25) (width 0.6) (layer F.Cu) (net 2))
 (segment (start 159.638 87.25) (end 157.48 89.408) (width 0.6) (layer F.Cu) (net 2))
 (segment (start 157.48 89.408) (end 157.48 94.488) (width 0.6) (layer F.Cu) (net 2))
 (segment (start 157.48 101.092) (end 157.48 108.204) (width 0.6) (layer F.Cu) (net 2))
 (segment (start 157.48 94.488) (end 157.48 101.092) (width 0.6) (layer F.Cu) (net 2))
 (segment (start 157.48 101.092) (end 158.878 102.49) (width 0.6) (layer F.Cu) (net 2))
 (segment (start 158.878 102.49) (end 161.684 102.49) (width 0.6) (layer F.Cu) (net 2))
 (segment (start 157.48 108.204) (end 159.386 110.11) (width 0.6) (layer F.Cu) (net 2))
 (segment (start 159.386 110.11) (end 161.684 110.11) (width 0.6) (layer F.Cu) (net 2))
 (segment (start 150.24 94.488) (end 157.48 94.488) (width 0.6) (layer F.Cu) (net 2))
 (segment (start 157.48 94.488) (end 161.302 94.488) (width 0.6) (layer F.Cu) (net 2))
 (segment (start 161.302 94.488) (end 161.684 94.87) (width 0.6) (layer F.Cu) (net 2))
 (segment (start 117.716 94.87) (end 117.476 94.87) (width 0.25) (layer F.Cu) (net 5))
 (segment (start 117.476 94.87) (end 113.156 90.55) (width 0.25) (layer F.Cu) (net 5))
 (segment (start 113.156 90.55) (end 112.916 90.55) (width 0.25) (layer F.Cu) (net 5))
 (segment (start 117.716 87.25) (end 117.716 87.008) (width 0.25) (layer F.Cu) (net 6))
 (segment (start 117.716 87.008) (end 118.11 86.614) (width 0.25) (layer F.Cu) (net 6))
 (segment (start 118.11 86.614) (end 121.986 86.614) (width 0.25) (layer F.Cu) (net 6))
 (segment (start 117.716 102.49) (end 117.476 102.49) (width 0.25) (layer F.Cu) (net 7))
 (segment (start 117.476 102.49) (end 113.156 98.17) (width 0.25) (layer F.Cu) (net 7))
 (segment (start 113.156 98.17) (end 112.916 98.17) (width 0.25) (layer F.Cu) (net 7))
 (segment (start 117.716 110.11) (end 117.222 110.11) (width 0.25) (layer F.Cu) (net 8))
 (segment (start 117.222 110.11) (end 112.916 105.804) (width 0.25) (layer F.Cu) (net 8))
 (segment (start 112.916 105.804) (end 112.916 105.79) (width 0.25) (layer F.Cu) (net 8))
 (segment (start 156.398 114.808) (end 161.236 114.808) (width 0.25) (layer F.Cu) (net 9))
 (segment (start 161.236 114.808) (end 161.684 114.36) (width 0.25) (layer F.Cu) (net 9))
 (segment (start 161.684 114.36) (end 161.684 113.41) (width 0.25) (layer F.Cu) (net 9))
 (segment (start 161.684 105.79) (end 161.884 105.79) (width 0.25) (layer F.Cu) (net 10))
 (segment (start 161.884 105.79) (end 166.204 110.11) (width 0.25) (layer F.Cu) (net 10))
 (segment (start 166.204 110.11) (end 166.484 110.11) (width 0.25) (layer F.Cu) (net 10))
 (segment (start 161.684 98.17) (end 161.684 98.184) (width 0.25) (layer F.Cu) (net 11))
 (segment (start 165.99 102.49) (end 166.484 102.49) (width 0.25) (layer F.Cu) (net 11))
 (segment (start 161.684 98.184) (end 165.99 102.49) (width 0.25) (layer F.Cu) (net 11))
 (segment (start 161.684 90.55) (end 161.884 90.55) (width 0.25) (layer F.Cu) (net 12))
 (segment (start 161.884 90.55) (end 166.204 94.87) (width 0.25) (layer F.Cu) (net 12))
 (segment (start 166.204 94.87) (end 166.484 94.87) (width 0.25) (layer F.Cu) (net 12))
 (segment (start 123.886 86.614) (end 125.476 86.614) (width 0.25) (layer F.Cu) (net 4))
 (segment (start 131.318 87.63) (end 136.652 87.63) (width 0.25) (layer F.Cu) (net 4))
 (segment (start 125.476 86.614) (end 127.254 88.392) (width 0.25) (layer F.Cu) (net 4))
 (segment (start 136.652 87.63) (end 141.372 92.35) (width 0.25) (layer F.Cu) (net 4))
 (segment (start 127.254 88.392) (end 130.556 88.392) (width 0.25) (layer F.Cu) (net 4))
 (segment (start 145.69 112.268) (end 146.94 112.268) (width 0.25) (layer F.Cu) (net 4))
 (segment (start 130.556 88.392) (end 131.318 87.63) (width 0.25) (layer F.Cu) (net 4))
 (segment (start 141.372 92.35) (end 141.372 107.95) (width 0.25) (layer F.Cu) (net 4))
 (segment (start 141.372 107.95) (end 145.69 112.268) (width 0.25) (layer F.Cu) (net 4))
 (segment (start 154.498 114.808) (end 150.24 114.808) (width 0.25) (layer F.Cu) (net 3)))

